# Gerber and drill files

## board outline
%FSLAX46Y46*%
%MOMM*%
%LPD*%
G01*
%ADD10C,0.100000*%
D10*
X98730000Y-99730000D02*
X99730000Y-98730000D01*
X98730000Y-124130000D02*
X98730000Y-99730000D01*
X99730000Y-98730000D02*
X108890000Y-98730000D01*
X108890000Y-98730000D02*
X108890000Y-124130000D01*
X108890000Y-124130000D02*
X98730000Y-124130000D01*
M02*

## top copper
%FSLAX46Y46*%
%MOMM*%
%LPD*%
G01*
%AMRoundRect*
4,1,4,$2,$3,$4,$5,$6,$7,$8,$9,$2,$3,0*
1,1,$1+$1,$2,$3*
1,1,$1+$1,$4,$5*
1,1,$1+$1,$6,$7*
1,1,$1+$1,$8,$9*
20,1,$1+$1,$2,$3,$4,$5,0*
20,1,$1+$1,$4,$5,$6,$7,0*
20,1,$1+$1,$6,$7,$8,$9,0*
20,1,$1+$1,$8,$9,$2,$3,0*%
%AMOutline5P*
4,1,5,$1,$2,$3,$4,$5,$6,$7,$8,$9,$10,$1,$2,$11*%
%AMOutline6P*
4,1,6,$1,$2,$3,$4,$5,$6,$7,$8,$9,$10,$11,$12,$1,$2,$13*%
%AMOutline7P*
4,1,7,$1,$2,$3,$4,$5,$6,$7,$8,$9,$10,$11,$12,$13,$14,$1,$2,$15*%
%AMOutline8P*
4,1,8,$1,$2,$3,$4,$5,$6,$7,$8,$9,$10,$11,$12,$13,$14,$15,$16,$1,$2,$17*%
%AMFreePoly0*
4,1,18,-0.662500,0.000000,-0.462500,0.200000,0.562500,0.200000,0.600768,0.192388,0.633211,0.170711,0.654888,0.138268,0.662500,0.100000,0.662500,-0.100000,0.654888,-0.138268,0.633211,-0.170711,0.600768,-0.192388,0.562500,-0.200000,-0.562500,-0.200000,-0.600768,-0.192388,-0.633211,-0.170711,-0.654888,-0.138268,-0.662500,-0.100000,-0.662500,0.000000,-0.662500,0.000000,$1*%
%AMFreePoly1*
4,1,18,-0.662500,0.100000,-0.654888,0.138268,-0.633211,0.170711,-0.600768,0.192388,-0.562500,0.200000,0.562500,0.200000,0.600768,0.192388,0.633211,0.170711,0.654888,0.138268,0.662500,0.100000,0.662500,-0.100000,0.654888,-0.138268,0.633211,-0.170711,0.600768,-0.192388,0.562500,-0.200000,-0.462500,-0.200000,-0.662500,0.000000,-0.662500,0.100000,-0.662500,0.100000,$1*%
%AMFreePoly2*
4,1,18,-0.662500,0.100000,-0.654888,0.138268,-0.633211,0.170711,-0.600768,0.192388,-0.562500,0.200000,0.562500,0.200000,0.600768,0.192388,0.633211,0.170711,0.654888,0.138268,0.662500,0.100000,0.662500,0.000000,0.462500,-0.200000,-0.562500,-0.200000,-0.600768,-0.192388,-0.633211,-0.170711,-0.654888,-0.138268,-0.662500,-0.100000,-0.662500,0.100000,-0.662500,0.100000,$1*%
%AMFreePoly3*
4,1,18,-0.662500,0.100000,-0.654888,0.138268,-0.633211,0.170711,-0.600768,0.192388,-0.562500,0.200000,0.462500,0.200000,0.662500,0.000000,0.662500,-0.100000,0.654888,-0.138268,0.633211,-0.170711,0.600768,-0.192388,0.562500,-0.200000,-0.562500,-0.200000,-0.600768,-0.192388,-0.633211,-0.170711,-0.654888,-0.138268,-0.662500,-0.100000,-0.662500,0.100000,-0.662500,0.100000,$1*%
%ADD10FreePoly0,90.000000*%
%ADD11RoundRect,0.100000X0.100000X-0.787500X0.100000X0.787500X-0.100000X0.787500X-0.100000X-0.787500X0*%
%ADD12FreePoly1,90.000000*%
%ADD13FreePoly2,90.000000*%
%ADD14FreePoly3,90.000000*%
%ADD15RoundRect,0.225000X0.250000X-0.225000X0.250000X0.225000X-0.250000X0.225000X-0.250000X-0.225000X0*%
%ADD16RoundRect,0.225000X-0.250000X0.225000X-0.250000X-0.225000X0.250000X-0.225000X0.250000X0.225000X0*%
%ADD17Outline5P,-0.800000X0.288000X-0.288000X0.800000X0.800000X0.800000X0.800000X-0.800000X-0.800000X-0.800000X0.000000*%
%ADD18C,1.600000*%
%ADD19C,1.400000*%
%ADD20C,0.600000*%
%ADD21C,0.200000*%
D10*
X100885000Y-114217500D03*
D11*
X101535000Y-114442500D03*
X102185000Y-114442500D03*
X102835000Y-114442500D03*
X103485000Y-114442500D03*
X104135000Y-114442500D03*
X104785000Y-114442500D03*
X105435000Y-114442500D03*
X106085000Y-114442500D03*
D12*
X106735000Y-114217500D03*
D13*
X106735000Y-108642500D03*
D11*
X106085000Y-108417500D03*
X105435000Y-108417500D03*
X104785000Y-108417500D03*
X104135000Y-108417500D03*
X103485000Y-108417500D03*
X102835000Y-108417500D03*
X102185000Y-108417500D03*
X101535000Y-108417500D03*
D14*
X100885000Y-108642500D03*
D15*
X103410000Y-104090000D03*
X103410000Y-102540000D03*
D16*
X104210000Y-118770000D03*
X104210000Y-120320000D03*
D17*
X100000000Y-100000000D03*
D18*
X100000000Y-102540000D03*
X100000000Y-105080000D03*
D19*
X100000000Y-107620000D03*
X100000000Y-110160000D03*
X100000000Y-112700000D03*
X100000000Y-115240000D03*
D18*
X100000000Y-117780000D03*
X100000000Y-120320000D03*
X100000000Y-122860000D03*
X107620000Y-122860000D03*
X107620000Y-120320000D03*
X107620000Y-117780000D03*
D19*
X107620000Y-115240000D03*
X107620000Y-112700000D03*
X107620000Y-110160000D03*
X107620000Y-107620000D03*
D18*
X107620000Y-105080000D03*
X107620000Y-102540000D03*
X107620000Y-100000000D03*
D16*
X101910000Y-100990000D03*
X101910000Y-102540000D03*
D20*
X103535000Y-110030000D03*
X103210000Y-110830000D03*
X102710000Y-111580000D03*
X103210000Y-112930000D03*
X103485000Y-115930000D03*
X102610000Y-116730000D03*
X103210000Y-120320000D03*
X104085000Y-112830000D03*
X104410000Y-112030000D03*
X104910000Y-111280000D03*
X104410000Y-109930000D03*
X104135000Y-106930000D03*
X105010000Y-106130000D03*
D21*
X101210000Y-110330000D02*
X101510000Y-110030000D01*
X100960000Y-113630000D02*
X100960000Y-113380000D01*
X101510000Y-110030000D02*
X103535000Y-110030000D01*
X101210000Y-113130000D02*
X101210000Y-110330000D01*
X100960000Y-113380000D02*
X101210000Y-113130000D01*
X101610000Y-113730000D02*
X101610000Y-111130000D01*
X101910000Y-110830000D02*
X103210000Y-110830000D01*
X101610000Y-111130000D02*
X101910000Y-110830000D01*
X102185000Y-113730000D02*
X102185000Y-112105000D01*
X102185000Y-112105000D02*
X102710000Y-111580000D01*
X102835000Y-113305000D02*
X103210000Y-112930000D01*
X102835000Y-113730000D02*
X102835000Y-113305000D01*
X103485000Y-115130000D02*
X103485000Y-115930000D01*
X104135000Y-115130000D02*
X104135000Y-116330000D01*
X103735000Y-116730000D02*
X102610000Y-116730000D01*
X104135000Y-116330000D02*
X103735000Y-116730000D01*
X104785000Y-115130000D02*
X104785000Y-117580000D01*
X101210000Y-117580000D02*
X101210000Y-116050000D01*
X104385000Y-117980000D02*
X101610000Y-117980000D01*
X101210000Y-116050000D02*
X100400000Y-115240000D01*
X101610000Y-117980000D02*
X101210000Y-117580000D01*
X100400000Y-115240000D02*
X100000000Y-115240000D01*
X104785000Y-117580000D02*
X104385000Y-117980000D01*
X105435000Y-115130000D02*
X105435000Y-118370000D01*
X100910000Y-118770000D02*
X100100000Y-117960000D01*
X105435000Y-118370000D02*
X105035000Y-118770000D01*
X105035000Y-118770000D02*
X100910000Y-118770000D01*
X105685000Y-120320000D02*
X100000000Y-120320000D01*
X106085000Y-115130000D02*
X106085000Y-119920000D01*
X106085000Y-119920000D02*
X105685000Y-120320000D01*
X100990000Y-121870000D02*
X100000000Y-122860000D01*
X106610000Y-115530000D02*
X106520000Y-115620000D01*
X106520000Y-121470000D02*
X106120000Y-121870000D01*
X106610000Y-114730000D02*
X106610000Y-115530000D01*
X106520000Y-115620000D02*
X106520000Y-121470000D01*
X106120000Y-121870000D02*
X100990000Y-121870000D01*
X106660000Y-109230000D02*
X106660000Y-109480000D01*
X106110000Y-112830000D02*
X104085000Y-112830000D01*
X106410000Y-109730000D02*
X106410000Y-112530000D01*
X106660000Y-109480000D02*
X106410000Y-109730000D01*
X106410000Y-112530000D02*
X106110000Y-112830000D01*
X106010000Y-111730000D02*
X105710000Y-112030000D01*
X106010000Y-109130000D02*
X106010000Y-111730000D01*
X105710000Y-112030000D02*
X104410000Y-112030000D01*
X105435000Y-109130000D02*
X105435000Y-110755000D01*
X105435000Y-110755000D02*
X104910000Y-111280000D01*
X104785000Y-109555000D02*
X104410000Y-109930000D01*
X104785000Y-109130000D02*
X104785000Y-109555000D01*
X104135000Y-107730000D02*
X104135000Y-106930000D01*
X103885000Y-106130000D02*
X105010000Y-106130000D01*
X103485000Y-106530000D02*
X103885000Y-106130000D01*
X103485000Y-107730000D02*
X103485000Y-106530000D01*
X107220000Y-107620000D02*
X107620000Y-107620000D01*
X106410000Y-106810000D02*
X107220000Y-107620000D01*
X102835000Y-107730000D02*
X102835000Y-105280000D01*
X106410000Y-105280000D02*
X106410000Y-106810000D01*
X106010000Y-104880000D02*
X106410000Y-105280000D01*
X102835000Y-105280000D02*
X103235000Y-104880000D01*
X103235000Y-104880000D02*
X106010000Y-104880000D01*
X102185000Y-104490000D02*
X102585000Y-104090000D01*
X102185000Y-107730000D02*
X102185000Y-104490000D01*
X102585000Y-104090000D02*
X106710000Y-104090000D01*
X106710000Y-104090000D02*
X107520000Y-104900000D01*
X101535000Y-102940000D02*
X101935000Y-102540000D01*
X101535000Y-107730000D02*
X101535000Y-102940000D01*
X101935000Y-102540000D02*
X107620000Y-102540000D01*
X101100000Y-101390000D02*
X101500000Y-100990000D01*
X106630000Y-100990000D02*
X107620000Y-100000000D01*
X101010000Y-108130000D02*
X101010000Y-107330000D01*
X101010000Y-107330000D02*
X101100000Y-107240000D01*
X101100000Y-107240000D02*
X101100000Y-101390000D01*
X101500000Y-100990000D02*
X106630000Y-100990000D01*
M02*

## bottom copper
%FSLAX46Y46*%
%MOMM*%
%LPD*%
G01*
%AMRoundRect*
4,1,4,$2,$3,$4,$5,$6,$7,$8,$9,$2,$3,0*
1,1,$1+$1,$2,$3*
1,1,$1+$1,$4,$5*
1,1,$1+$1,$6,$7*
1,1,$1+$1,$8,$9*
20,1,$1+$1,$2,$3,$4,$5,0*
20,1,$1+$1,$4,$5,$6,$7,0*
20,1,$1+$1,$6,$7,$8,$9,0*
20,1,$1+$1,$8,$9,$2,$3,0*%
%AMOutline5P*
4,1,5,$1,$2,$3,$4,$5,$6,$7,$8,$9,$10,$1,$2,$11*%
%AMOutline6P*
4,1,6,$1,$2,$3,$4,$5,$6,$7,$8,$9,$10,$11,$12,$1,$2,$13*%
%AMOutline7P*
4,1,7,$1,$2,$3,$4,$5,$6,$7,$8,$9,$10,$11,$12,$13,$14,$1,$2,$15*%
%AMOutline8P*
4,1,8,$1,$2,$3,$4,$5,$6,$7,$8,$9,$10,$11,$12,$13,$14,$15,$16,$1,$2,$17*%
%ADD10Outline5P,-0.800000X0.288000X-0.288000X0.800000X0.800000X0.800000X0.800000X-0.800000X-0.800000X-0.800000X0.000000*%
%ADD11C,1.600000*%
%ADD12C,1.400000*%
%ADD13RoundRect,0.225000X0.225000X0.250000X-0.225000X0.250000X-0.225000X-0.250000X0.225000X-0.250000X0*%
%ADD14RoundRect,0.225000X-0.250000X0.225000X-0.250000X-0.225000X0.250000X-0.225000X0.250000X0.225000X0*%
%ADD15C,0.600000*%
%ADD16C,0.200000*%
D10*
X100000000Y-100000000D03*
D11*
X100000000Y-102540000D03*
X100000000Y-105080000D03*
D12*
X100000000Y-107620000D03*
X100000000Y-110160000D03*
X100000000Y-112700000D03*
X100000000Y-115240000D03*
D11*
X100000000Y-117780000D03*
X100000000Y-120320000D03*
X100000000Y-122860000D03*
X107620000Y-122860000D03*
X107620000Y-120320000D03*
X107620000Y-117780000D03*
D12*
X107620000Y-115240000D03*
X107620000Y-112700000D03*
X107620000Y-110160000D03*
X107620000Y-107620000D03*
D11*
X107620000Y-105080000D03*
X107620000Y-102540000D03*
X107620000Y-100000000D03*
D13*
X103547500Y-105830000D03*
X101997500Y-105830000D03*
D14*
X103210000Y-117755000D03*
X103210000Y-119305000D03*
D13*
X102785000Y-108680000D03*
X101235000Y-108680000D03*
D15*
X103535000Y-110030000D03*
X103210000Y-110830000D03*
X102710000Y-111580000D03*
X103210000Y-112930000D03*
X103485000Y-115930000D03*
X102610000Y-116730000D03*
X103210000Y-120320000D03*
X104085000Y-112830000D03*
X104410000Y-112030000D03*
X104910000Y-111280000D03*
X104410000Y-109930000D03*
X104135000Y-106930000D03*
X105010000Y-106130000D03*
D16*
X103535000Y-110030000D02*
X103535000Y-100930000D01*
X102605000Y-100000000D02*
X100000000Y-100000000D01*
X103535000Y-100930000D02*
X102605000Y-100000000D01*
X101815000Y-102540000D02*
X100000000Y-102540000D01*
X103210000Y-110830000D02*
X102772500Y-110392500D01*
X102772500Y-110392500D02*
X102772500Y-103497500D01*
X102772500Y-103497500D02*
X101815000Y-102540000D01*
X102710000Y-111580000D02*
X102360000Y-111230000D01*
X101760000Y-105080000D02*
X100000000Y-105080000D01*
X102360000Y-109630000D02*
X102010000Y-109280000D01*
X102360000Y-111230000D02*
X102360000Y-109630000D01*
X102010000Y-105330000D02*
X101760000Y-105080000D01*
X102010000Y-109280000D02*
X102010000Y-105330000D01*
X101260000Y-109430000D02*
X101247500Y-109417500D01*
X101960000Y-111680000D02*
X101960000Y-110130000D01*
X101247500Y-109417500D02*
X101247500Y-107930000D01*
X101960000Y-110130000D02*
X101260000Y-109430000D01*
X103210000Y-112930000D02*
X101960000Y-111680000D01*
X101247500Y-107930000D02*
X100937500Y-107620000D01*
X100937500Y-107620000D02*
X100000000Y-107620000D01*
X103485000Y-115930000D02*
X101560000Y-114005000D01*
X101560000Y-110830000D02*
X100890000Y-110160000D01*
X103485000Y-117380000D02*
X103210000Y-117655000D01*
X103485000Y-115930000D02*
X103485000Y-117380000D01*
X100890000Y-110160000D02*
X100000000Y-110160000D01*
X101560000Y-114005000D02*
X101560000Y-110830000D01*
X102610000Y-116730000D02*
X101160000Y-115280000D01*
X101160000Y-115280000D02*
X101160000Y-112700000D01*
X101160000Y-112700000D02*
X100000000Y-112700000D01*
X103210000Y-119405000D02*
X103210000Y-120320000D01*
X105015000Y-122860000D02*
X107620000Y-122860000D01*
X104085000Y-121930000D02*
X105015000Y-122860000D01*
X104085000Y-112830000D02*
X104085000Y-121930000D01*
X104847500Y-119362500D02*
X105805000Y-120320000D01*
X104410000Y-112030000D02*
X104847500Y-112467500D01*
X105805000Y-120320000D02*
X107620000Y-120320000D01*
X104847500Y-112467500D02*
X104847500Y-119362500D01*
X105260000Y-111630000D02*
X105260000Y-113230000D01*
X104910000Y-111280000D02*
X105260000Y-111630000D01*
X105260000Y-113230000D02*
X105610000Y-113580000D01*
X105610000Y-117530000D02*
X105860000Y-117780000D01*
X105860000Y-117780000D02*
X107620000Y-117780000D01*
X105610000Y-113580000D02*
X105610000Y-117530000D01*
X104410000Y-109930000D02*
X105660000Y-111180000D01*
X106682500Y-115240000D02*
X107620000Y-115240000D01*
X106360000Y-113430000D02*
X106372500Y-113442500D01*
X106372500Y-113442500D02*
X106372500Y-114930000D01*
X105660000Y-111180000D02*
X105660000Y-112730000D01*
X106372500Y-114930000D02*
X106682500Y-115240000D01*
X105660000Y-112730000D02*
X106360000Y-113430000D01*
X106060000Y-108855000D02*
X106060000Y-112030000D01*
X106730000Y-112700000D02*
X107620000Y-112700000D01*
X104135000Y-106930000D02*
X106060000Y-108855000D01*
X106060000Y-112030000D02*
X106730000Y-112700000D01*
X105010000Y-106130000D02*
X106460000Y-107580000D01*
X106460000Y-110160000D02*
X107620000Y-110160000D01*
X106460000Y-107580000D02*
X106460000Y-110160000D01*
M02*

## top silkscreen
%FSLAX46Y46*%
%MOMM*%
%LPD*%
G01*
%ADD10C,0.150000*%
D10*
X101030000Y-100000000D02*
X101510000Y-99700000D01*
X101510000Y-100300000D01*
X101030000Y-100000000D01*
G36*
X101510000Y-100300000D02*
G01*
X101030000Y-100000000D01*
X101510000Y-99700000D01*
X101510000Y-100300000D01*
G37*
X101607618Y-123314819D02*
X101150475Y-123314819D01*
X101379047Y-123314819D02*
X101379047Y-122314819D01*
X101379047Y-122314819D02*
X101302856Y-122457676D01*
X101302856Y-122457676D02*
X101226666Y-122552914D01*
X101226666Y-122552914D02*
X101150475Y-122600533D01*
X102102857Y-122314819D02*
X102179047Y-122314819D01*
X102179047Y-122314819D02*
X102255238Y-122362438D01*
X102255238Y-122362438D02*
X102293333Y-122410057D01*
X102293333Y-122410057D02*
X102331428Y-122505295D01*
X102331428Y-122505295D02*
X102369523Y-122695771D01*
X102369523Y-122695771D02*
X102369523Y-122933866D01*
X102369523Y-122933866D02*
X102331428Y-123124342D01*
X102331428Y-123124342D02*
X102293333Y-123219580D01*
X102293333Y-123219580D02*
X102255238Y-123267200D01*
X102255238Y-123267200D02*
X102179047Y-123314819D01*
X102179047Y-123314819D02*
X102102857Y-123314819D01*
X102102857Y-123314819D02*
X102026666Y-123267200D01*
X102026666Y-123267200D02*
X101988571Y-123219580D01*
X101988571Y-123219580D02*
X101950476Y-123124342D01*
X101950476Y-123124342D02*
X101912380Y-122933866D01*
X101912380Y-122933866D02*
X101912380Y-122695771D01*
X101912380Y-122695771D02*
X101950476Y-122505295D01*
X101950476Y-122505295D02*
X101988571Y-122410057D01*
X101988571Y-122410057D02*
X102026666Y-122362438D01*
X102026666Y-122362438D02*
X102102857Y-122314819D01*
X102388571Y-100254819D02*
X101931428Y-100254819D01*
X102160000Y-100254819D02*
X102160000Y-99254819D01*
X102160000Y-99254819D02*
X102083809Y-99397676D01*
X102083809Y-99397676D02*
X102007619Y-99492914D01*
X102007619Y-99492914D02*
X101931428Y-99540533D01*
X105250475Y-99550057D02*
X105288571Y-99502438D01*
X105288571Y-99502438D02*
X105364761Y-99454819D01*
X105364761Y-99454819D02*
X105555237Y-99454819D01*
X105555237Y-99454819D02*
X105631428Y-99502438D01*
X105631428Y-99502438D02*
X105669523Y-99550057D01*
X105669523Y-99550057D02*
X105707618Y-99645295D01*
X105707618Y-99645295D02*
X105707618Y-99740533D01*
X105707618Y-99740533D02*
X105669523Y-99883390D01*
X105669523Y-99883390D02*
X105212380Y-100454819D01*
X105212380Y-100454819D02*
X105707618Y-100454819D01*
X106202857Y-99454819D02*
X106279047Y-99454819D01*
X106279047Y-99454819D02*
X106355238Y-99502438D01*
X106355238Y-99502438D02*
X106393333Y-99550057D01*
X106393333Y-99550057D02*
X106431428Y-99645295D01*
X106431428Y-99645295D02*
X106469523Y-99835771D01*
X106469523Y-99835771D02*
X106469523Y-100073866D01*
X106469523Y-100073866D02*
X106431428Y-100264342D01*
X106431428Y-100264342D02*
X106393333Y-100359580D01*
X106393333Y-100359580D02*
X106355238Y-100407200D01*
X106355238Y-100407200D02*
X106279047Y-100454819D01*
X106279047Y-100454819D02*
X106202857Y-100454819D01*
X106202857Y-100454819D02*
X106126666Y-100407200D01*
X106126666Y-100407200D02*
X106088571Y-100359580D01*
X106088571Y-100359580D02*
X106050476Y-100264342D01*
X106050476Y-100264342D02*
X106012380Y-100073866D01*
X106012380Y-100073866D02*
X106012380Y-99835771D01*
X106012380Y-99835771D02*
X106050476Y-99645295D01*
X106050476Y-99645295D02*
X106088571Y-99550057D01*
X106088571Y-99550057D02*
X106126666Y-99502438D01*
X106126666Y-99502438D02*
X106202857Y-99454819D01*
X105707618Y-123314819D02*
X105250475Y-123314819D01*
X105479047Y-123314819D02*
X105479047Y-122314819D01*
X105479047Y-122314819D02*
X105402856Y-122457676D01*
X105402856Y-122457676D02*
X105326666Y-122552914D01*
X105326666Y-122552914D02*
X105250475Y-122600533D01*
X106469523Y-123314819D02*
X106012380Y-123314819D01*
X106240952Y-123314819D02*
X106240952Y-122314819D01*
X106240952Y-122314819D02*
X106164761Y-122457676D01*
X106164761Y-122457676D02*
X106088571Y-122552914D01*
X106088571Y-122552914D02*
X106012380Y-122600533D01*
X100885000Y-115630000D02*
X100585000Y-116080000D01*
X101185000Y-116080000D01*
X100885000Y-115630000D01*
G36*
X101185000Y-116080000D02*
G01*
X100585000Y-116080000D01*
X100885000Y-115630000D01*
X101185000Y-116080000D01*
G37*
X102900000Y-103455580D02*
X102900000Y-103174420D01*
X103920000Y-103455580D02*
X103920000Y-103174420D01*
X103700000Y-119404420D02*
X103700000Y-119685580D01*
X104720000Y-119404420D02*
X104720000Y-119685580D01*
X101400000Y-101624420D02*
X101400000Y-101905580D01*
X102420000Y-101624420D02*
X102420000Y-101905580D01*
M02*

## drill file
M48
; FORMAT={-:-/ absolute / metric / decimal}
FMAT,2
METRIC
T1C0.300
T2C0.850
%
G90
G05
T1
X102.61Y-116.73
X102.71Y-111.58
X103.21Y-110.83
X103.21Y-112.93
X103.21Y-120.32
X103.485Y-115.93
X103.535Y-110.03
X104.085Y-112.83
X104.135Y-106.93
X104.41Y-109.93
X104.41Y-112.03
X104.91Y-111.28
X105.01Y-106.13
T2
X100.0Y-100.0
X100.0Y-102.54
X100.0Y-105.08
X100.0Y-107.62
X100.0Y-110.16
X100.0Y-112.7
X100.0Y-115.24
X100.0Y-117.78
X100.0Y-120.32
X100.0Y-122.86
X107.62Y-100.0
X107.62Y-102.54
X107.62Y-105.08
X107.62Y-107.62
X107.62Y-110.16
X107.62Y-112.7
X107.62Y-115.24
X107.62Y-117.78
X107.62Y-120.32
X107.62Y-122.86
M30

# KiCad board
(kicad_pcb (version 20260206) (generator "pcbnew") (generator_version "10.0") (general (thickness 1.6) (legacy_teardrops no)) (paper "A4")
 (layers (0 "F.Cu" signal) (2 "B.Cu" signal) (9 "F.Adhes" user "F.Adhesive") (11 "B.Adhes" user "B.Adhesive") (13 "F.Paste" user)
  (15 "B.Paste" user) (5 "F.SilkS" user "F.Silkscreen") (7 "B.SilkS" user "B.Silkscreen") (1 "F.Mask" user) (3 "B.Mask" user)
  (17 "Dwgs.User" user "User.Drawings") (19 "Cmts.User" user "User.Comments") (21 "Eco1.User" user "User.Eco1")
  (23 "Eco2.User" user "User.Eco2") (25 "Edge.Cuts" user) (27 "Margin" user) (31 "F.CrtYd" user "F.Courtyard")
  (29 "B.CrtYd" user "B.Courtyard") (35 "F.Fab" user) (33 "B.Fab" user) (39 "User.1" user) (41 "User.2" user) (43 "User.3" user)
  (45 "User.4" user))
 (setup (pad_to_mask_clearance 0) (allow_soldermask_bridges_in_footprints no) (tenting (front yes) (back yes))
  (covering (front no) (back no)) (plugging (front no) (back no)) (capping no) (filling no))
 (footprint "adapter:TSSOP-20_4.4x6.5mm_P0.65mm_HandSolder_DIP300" (layer "F.Cu") (at 103.81 111.43 90)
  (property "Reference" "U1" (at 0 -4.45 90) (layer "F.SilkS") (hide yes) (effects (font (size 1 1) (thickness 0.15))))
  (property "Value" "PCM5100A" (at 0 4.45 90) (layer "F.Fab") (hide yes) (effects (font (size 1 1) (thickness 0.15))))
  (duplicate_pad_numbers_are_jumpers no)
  (fp_poly (pts (xy -4.2 -2.925) (xy -4.65 -3.225) (xy -4.65 -2.625)) (stroke (width 0.15) (type solid)) (fill yes) (layer "F.SilkS"))
  (pad "1" smd roundrect (at -2.7875 -2.925 90) (size 1.325 0.4) (layers "F.Cu" "F.Mask" "F.Paste") (roundrect_rratio 0.25)
   (chamfer_ratio 0.5) (chamfer top_left) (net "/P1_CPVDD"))
  (pad "2" smd roundrect (at -3.0125 -2.275 90) (size 1.775 0.4) (layers "F.Cu" "F.Mask" "F.Paste") (roundrect_rratio 0.25) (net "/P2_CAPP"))
  (pad "3" smd roundrect (at -3.0125 -1.625 90) (size 1.775 0.4) (layers "F.Cu" "F.Mask" "F.Paste") (roundrect_rratio 0.25)
   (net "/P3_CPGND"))
  (pad "4" smd roundrect (at -3.0125 -0.975 90) (size 1.775 0.4) (layers "F.Cu" "F.Mask" "F.Paste") (roundrect_rratio 0.25) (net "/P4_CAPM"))
  (pad "5" smd roundrect (at -3.0125 -0.325 90) (size 1.775 0.4) (layers "F.Cu" "F.Mask" "F.Paste") (roundrect_rratio 0.25) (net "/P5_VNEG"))
  (pad "6" smd roundrect (at -3.0125 0.325 90) (size 1.775 0.4) (layers "F.Cu" "F.Mask" "F.Paste") (roundrect_rratio 0.25) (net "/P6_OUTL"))
  (pad "7" smd roundrect (at -3.0125 0.975 90) (size 1.775 0.4) (layers "F.Cu" "F.Mask" "F.Paste") (roundrect_rratio 0.25) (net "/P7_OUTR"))
  (pad "8" smd roundrect (at -3.0125 1.625 90) (size 1.775 0.4) (layers "F.Cu" "F.Mask" "F.Paste") (roundrect_rratio 0.25) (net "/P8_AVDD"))
  (pad "9" smd roundrect (at -3.0125 2.275 90) (size 1.775 0.4) (layers "F.Cu" "F.Mask" "F.Paste") (roundrect_rratio 0.25) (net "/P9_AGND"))
  (pad "10" smd roundrect (at -2.7875 2.925 90) (size 1.325 0.4) (layers "F.Cu" "F.Mask" "F.Paste") (roundrect_rratio 0.25)
   (chamfer_ratio 0.5) (chamfer bottom_left) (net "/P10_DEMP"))
  (pad "11" smd roundrect (at 2.7875 2.925 90) (size 1.325 0.4) (layers "F.Cu" "F.Mask" "F.Paste") (roundrect_rratio 0.25)
   (chamfer_ratio 0.5) (chamfer bottom_right) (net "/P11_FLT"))
  (pad "12" smd roundrect (at 3.0125 2.275 90) (size 1.775 0.4) (layers "F.Cu" "F.Mask" "F.Paste") (roundrect_rratio 0.25) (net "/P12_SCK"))
  (pad "13" smd roundrect (at 3.0125 1.625 90) (size 1.775 0.4) (layers "F.Cu" "F.Mask" "F.Paste") (roundrect_rratio 0.25) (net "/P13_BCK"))
  (pad "14" smd roundrect (at 3.0125 0.975 90) (size 1.775 0.4) (layers "F.Cu" "F.Mask" "F.Paste") (roundrect_rratio 0.25) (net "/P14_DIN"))
  (pad "15" smd roundrect (at 3.0125 0.325 90) (size 1.775 0.4) (layers "F.Cu" "F.Mask" "F.Paste") (roundrect_rratio 0.25) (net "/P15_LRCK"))
  (pad "16" smd roundrect (at 3.0125 -0.325 90) (size 1.775 0.4) (layers "F.Cu" "F.Mask" "F.Paste") (roundrect_rratio 0.25) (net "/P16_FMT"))
  (pad "17" smd roundrect (at 3.0125 -0.975 90) (size 1.775 0.4) (layers "F.Cu" "F.Mask" "F.Paste") (roundrect_rratio 0.25)
   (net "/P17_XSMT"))
  (pad "18" smd roundrect (at 3.0125 -1.625 90) (size 1.775 0.4) (layers "F.Cu" "F.Mask" "F.Paste") (roundrect_rratio 0.25)
   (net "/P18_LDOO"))
  (pad "19" smd roundrect (at 3.0125 -2.275 90) (size 1.775 0.4) (layers "F.Cu" "F.Mask" "F.Paste") (roundrect_rratio 0.25)
   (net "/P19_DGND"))
  (pad "20" smd roundrect (at 2.7875 -2.925 90) (size 1.325 0.4) (layers "F.Cu" "F.Mask" "F.Paste") (roundrect_rratio 0.25)
   (chamfer_ratio 0.5) (chamfer top_right) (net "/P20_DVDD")))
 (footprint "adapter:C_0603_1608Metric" (layer "F.Cu") (at 103.41 103.315 90)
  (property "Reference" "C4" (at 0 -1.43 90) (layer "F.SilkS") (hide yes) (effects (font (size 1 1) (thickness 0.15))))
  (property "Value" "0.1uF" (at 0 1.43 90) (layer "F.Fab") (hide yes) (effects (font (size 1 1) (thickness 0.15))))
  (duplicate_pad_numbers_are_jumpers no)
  (fp_line (start -0.14058 -0.51) (end 0.14058 -0.51) (stroke (width 0.15) (type solid)) (layer "F.SilkS"))
  (fp_line (start -0.14058 0.51) (end 0.14058 0.51) (stroke (width 0.15) (type solid)) (layer "F.SilkS"))
  (pad "1" smd roundrect (at -0.775 0 90) (size 0.9 0.95) (layers "F.Cu" "F.Mask" "F.Paste") (roundrect_rratio 0.25) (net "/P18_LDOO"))
  (pad "2" smd roundrect (at 0.775 0 90) (size 0.9 0.95) (layers "F.Cu" "F.Mask" "F.Paste") (roundrect_rratio 0.25) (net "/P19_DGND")))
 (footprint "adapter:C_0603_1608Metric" (layer "F.Cu") (at 104.21 119.545 -90)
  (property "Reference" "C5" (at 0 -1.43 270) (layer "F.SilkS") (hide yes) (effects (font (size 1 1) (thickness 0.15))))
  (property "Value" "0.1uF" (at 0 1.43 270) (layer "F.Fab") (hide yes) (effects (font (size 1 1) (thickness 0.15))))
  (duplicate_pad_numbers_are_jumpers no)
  (fp_line (start -0.14058 0.51) (end 0.14058 0.51) (stroke (width 0.15) (type solid)) (layer "F.SilkS"))
  (fp_line (start -0.14058 -0.51) (end 0.14058 -0.51) (stroke (width 0.15) (type solid)) (layer "F.SilkS"))
  (pad "1" smd roundrect (at -0.775 0 270) (size 0.9 0.95) (layers "F.Cu" "F.Mask" "F.Paste") (roundrect_rratio 0.25) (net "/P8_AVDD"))
  (pad "2" smd roundrect (at 0.775 0 270) (size 0.9 0.95) (layers "F.Cu" "F.Mask" "F.Paste") (roundrect_rratio 0.25) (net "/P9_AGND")))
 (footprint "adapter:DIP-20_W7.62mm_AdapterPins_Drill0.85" (layer "F.Cu") (at 100 100)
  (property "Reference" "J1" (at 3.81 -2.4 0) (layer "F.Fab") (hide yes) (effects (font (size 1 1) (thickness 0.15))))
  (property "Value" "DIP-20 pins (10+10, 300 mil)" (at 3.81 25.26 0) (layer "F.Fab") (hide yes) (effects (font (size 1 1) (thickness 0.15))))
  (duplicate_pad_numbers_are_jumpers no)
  (pad "1" thru_hole roundrect (at 0 0) (size 1.6 1.6) (drill 0.85) (layers "*.Cu" "*.Mask") (remove_unused_layers no) (roundrect_rratio 0)
   (chamfer_ratio 0.32) (chamfer top_left) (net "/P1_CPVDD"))
  (pad "2" thru_hole circle (at 0 2.54) (size 1.6 1.6) (drill 0.85) (layers "*.Cu" "*.Mask") (remove_unused_layers no) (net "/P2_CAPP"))
  (pad "3" thru_hole circle (at 0 5.08) (size 1.6 1.6) (drill 0.85) (layers "*.Cu" "*.Mask") (remove_unused_layers no) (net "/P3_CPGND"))
  (pad "4" thru_hole circle (at 0 7.62) (size 1.4 1.4) (drill 0.85) (layers "*.Cu" "*.Mask") (remove_unused_layers no) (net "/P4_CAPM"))
  (pad "5" thru_hole circle (at 0 10.16) (size 1.4 1.4) (drill 0.85) (layers "*.Cu" "*.Mask") (remove_unused_layers no) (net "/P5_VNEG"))
  (pad "6" thru_hole circle (at 0 12.7) (size 1.4 1.4) (drill 0.85) (layers "*.Cu" "*.Mask") (remove_unused_layers no) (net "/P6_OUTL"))
  (pad "7" thru_hole circle (at 0 15.24) (size 1.4 1.4) (drill 0.85) (layers "*.Cu" "*.Mask") (remove_unused_layers no) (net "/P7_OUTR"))
  (pad "8" thru_hole circle (at 0 17.78) (size 1.6 1.6) (drill 0.85) (layers "*.Cu" "*.Mask") (remove_unused_layers no) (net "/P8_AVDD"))
  (pad "9" thru_hole circle (at 0 20.32) (size 1.6 1.6) (drill 0.85) (layers "*.Cu" "*.Mask") (remove_unused_layers no) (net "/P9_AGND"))
  (pad "10" thru_hole circle (at 0 22.86) (size 1.6 1.6) (drill 0.85) (layers "*.Cu" "*.Mask") (remove_unused_layers no) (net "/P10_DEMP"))
  (pad "11" thru_hole circle (at 7.62 22.86) (size 1.6 1.6) (drill 0.85) (layers "*.Cu" "*.Mask") (remove_unused_layers no) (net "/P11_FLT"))
  (pad "12" thru_hole circle (at 7.62 20.32) (size 1.6 1.6) (drill 0.85) (layers "*.Cu" "*.Mask") (remove_unused_layers no) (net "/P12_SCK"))
  (pad "13" thru_hole circle (at 7.62 17.78) (size 1.6 1.6) (drill 0.85) (layers "*.Cu" "*.Mask") (remove_unused_layers no) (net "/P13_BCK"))
  (pad "14" thru_hole circle (at 7.62 15.24) (size 1.4 1.4) (drill 0.85) (layers "*.Cu" "*.Mask") (remove_unused_layers no) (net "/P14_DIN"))
  (pad "15" thru_hole circle (at 7.62 12.7) (size 1.4 1.4) (drill 0.85) (layers "*.Cu" "*.Mask") (remove_unused_layers no) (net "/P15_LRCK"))
  (pad "16" thru_hole circle (at 7.62 10.16) (size 1.4 1.4) (drill 0.85) (layers "*.Cu" "*.Mask") (remove_unused_layers no) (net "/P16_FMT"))
  (pad "17" thru_hole circle (at 7.62 7.62) (size 1.4 1.4) (drill 0.85) (layers "*.Cu" "*.Mask") (remove_unused_layers no) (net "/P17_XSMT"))
  (pad "18" thru_hole circle (at 7.62 5.08) (size 1.6 1.6) (drill 0.85) (layers "*.Cu" "*.Mask") (remove_unused_layers no) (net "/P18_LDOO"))
  (pad "19" thru_hole circle (at 7.62 2.54) (size 1.6 1.6) (drill 0.85) (layers "*.Cu" "*.Mask") (remove_unused_layers no) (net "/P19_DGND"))
  (pad "20" thru_hole circle (at 7.62 0) (size 1.6 1.6) (drill 0.85) (layers "*.Cu" "*.Mask") (remove_unused_layers no) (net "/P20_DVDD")))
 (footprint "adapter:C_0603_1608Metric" (layer "F.Cu") (at 101.91 101.765 -90)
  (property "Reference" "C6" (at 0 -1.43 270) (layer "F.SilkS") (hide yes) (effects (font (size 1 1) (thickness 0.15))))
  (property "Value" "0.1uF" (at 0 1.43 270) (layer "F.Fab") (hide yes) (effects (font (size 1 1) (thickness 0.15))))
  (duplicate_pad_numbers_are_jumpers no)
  (fp_line (start -0.14058 0.51) (end 0.14058 0.51) (stroke (width 0.15) (type solid)) (layer "F.SilkS"))
  (fp_line (start -0.14058 -0.51) (end 0.14058 -0.51) (stroke (width 0.15) (type solid)) (layer "F.SilkS"))
  (pad "1" smd roundrect (at -0.775 0 270) (size 0.9 0.95) (layers "F.Cu" "F.Mask" "F.Paste") (roundrect_rratio 0.25) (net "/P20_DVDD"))
  (pad "2" smd roundrect (at 0.775 0 270) (size 0.9 0.95) (layers "F.Cu" "F.Mask" "F.Paste") (roundrect_rratio 0.25) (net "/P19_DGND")))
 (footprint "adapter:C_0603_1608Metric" (layer "B.Cu") (at 102.7725 105.83 180)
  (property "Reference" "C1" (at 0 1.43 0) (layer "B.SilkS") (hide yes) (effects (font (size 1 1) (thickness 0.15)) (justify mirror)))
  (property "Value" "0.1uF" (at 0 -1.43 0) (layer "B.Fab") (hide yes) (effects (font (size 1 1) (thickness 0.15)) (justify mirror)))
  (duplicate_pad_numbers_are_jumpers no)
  (pad "1" smd roundrect (at -0.775 0 180) (size 0.9 0.95) (layers "B.Cu" "B.Mask" "B.Paste") (roundrect_rratio 0.25) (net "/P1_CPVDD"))
  (pad "2" smd roundrect (at 0.775 0 180) (size 0.9 0.95) (layers "B.Cu" "B.Mask" "B.Paste") (roundrect_rratio 0.25) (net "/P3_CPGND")))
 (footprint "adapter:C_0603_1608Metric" (layer "B.Cu") (at 103.21 118.53 -90)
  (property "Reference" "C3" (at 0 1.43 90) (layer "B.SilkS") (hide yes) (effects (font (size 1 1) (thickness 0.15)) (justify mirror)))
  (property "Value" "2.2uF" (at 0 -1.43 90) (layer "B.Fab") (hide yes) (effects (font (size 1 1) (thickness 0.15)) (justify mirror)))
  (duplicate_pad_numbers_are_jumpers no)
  (pad "1" smd roundrect (at -0.775 0 270) (size 0.9 0.95) (layers "B.Cu" "B.Mask" "B.Paste") (roundrect_rratio 0.25) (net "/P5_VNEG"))
  (pad "2" smd roundrect (at 0.775 0 270) (size 0.9 0.95) (layers "B.Cu" "B.Mask" "B.Paste") (roundrect_rratio 0.25) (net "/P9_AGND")))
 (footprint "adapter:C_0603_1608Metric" (layer "B.Cu") (at 102.01 108.68 180)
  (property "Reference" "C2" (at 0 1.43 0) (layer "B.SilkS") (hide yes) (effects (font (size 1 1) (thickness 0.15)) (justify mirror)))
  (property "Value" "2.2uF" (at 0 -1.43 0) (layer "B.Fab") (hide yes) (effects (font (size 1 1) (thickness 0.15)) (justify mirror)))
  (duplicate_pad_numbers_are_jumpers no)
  (pad "1" smd roundrect (at -0.775 0 180) (size 0.9 0.95) (layers "B.Cu" "B.Mask" "B.Paste") (roundrect_rratio 0.25) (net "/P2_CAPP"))
  (pad "2" smd roundrect (at 0.775 0 180) (size 0.9 0.95) (layers "B.Cu" "B.Mask" "B.Paste") (roundrect_rratio 0.25) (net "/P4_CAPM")))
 (gr_poly (pts (xy 101.03 100) (xy 101.51 99.7) (xy 101.51 100.3)) (stroke (width 0.15) (type default)) (fill yes) (layer "F.SilkS"))
 (gr_line (start 98.73 99.73) (end 99.73 98.73) (stroke (width 0.1) (type default)) (layer "Edge.Cuts"))
 (gr_line (start 98.73 124.13) (end 98.73 99.73) (stroke (width 0.1) (type default)) (layer "Edge.Cuts"))
 (gr_line (start 99.73 98.73) (end 108.89 98.73) (stroke (width 0.1) (type default)) (layer "Edge.Cuts"))
 (gr_line (start 108.89 98.73) (end 108.89 124.13) (stroke (width 0.1) (type default)) (layer "Edge.Cuts"))
 (gr_line (start 108.89 124.13) (end 98.73 124.13) (stroke (width 0.1) (type default)) (layer "Edge.Cuts"))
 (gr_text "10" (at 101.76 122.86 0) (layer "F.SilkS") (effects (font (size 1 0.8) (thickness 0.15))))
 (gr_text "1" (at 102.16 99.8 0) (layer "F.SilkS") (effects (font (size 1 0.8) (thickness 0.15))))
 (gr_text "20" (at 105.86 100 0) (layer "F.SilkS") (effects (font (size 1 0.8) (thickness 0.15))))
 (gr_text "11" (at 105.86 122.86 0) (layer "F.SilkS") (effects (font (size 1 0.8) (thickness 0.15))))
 (segment (start 101.21 110.33) (end 101.51 110.03) (width 0.2) (layer "F.Cu") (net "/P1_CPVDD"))
 (segment (start 100.96 113.63) (end 100.96 113.38) (width 0.2) (layer "F.Cu") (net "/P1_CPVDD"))
 (segment (start 101.51 110.03) (end 103.535 110.03) (width 0.2) (layer "F.Cu") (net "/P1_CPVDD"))
 (segment (start 101.21 113.13) (end 101.21 110.33) (width 0.2) (layer "F.Cu") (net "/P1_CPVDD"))
 (segment (start 100.96 113.38) (end 101.21 113.13) (width 0.2) (layer "F.Cu") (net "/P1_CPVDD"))
 (via (at 103.535 110.03) (size 0.6) (drill 0.3) (layers "F.Cu" "B.Cu") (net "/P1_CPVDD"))
 (segment (start 103.535 110.03) (end 103.535 100.93) (width 0.2) (layer "B.Cu") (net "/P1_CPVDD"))
 (segment (start 102.605 100) (end 100 100) (width 0.2) (layer "B.Cu") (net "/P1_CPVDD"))
 (segment (start 103.535 100.93) (end 102.605 100) (width 0.2) (layer "B.Cu") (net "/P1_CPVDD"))
 (segment (start 101.61 113.73) (end 101.61 111.13) (width 0.2) (layer "F.Cu") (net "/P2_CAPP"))
 (segment (start 101.91 110.83) (end 103.21 110.83) (width 0.2) (layer "F.Cu") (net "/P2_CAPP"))
 (segment (start 101.61 111.13) (end 101.91 110.83) (width 0.2) (layer "F.Cu") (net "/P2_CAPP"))
 (via (at 103.21 110.83) (size 0.6) (drill 0.3) (layers "F.Cu" "B.Cu") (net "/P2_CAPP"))
 (segment (start 101.815 102.54) (end 100 102.54) (width 0.2) (layer "B.Cu") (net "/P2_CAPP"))
 (segment (start 103.21 110.83) (end 102.7725 110.3925) (width 0.2) (layer "B.Cu") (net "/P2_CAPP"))
 (segment (start 102.7725 110.3925) (end 102.7725 103.4975) (width 0.2) (layer "B.Cu") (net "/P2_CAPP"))
 (segment (start 102.7725 103.4975) (end 101.815 102.54) (width 0.2) (layer "B.Cu") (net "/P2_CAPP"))
 (segment (start 102.185 113.73) (end 102.185 112.105) (width 0.2) (layer "F.Cu") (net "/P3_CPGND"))
 (segment (start 102.185 112.105) (end 102.71 111.58) (width 0.2) (layer "F.Cu") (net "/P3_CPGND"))
 (via (at 102.71 111.58) (size 0.6) (drill 0.3) (layers "F.Cu" "B.Cu") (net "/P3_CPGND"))
 (segment (start 102.71 111.58) (end 102.36 111.23) (width 0.2) (layer "B.Cu") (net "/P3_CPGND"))
 (segment (start 101.76 105.08) (end 100 105.08) (width 0.2) (layer "B.Cu") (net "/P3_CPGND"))
 (segment (start 102.36 109.63) (end 102.01 109.28) (width 0.2) (layer "B.Cu") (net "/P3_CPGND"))
 (segment (start 102.36 111.23) (end 102.36 109.63) (width 0.2) (layer "B.Cu") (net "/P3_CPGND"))
 (segment (start 102.01 105.33) (end 101.76 105.08) (width 0.2) (layer "B.Cu") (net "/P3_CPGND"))
 (segment (start 102.01 109.28) (end 102.01 105.33) (width 0.2) (layer "B.Cu") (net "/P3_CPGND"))
 (segment (start 102.835 113.305) (end 103.21 112.93) (width 0.2) (layer "F.Cu") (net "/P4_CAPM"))
 (segment (start 102.835 113.73) (end 102.835 113.305) (width 0.2) (layer "F.Cu") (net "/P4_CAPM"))
 (via (at 103.21 112.93) (size 0.6) (drill 0.3) (layers "F.Cu" "B.Cu") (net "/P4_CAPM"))
 (segment (start 101.26 109.43) (end 101.2475 109.4175) (width 0.2) (layer "B.Cu") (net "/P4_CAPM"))
 (segment (start 101.96 111.68) (end 101.96 110.13) (width 0.2) (layer "B.Cu") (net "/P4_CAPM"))
 (segment (start 101.2475 109.4175) (end 101.2475 107.93) (width 0.2) (layer "B.Cu") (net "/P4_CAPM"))
 (segment (start 101.96 110.13) (end 101.26 109.43) (width 0.2) (layer "B.Cu") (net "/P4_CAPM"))
 (segment (start 103.21 112.93) (end 101.96 111.68) (width 0.2) (layer "B.Cu") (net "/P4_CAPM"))
 (segment (start 101.2475 107.93) (end 100.9375 107.62) (width 0.2) (layer "B.Cu") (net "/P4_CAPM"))
 (segment (start 100.9375 107.62) (end 100 107.62) (width 0.2) (layer "B.Cu") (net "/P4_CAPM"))
 (segment (start 103.485 115.13) (end 103.485 115.93) (width 0.2) (layer "F.Cu") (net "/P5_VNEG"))
 (via (at 103.485 115.93) (size 0.6) (drill 0.3) (layers "F.Cu" "B.Cu") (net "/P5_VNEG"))
 (segment (start 103.485 115.93) (end 101.56 114.005) (width 0.2) (layer "B.Cu") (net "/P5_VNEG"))
 (segment (start 101.56 110.83) (end 100.89 110.16) (width 0.2) (layer "B.Cu") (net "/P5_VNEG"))
 (segment (start 103.485 117.38) (end 103.21 117.655) (width 0.2) (layer "B.Cu") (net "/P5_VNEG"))
 (segment (start 103.485 115.93) (end 103.485 117.38) (width 0.2) (layer "B.Cu") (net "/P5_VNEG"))
 (segment (start 100.89 110.16) (end 100 110.16) (width 0.2) (layer "B.Cu") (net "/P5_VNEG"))
 (segment (start 101.56 114.005) (end 101.56 110.83) (width 0.2) (layer "B.Cu") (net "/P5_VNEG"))
 (segment (start 104.135 115.13) (end 104.135 116.33) (width 0.2) (layer "F.Cu") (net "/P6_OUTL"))
 (segment (start 103.735 116.73) (end 102.61 116.73) (width 0.2) (layer "F.Cu") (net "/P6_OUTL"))
 (segment (start 104.135 116.33) (end 103.735 116.73) (width 0.2) (layer "F.Cu") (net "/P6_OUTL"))
 (via (at 102.61 116.73) (size 0.6) (drill 0.3) (layers "F.Cu" "B.Cu") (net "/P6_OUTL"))
 (segment (start 102.61 116.73) (end 101.16 115.28) (width 0.2) (layer "B.Cu") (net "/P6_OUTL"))
 (segment (start 101.16 115.28) (end 101.16 112.7) (width 0.2) (layer "B.Cu") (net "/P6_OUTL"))
 (segment (start 101.16 112.7) (end 100 112.7) (width 0.2) (layer "B.Cu") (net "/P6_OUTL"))
 (segment (start 104.785 115.13) (end 104.785 117.58) (width 0.2) (layer "F.Cu") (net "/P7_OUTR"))
 (segment (start 101.21 117.58) (end 101.21 116.05) (width 0.2) (layer "F.Cu") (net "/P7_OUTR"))
 (segment (start 104.385 117.98) (end 101.61 117.98) (width 0.2) (layer "F.Cu") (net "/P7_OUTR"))
 (segment (start 101.21 116.05) (end 100.4 115.24) (width 0.2) (layer "F.Cu") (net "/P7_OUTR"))
 (segment (start 101.61 117.98) (end 101.21 117.58) (width 0.2) (layer "F.Cu") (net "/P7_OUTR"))
 (segment (start 100.4 115.24) (end 100 115.24) (width 0.2) (layer "F.Cu") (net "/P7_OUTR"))
 (segment (start 104.785 117.58) (end 104.385 117.98) (width 0.2) (layer "F.Cu") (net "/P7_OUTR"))
 (segment (start 105.435 115.13) (end 105.435 118.37) (width 0.2) (layer "F.Cu") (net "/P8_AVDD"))
 (segment (start 100.91 118.77) (end 100.1 117.96) (width 0.2) (layer "F.Cu") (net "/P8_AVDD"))
 (segment (start 105.435 118.37) (end 105.035 118.77) (width 0.2) (layer "F.Cu") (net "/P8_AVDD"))
 (segment (start 105.035 118.77) (end 100.91 118.77) (width 0.2) (layer "F.Cu") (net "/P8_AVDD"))
 (segment (start 105.685 120.32) (end 100 120.32) (width 0.2) (layer "F.Cu") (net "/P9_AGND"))
 (segment (start 106.085 115.13) (end 106.085 119.92) (width 0.2) (layer "F.Cu") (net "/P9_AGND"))
 (segment (start 106.085 119.92) (end 105.685 120.32) (width 0.2) (layer "F.Cu") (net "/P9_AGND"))
 (via (at 103.21 120.32) (size 0.6) (drill 0.3) (layers "F.Cu" "B.Cu") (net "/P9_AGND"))
 (segment (start 103.21 119.405) (end 103.21 120.32) (width 0.2) (layer "B.Cu") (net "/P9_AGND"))
 (segment (start 100.99 121.87) (end 100 122.86) (width 0.2) (layer "F.Cu") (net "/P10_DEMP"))
 (segment (start 106.61 115.53) (end 106.52 115.62) (width 0.2) (layer "F.Cu") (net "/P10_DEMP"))
 (segment (start 106.52 121.47) (end 106.12 121.87) (width 0.2) (layer "F.Cu") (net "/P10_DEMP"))
 (segment (start 106.61 114.73) (end 106.61 115.53) (width 0.2) (layer "F.Cu") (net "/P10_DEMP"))
 (segment (start 106.52 115.62) (end 106.52 121.47) (width 0.2) (layer "F.Cu") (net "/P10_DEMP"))
 (segment (start 106.12 121.87) (end 100.99 121.87) (width 0.2) (layer "F.Cu") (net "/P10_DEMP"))
 (segment (start 106.66 109.23) (end 106.66 109.48) (width 0.2) (layer "F.Cu") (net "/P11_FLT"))
 (segment (start 106.11 112.83) (end 104.085 112.83) (width 0.2) (layer "F.Cu") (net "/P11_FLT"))
 (segment (start 106.41 109.73) (end 106.41 112.53) (width 0.2) (layer "F.Cu") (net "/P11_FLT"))
 (segment (start 106.66 109.48) (end 106.41 109.73) (width 0.2) (layer "F.Cu") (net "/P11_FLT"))
 (segment (start 106.41 112.53) (end 106.11 112.83) (width 0.2) (layer "F.Cu") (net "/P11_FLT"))
 (via (at 104.085 112.83) (size 0.6) (drill 0.3) (layers "F.Cu" "B.Cu") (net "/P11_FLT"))
 (segment (start 105.015 122.86) (end 107.62 122.86) (width 0.2) (layer "B.Cu") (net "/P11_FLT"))
 (segment (start 104.085 121.93) (end 105.015 122.86) (width 0.2) (layer "B.Cu") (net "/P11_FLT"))
 (segment (start 104.085 112.83) (end 104.085 121.93) (width 0.2) (layer "B.Cu") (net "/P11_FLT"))
 (segment (start 106.01 111.73) (end 105.71 112.03) (width 0.2) (layer "F.Cu") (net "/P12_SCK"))
 (segment (start 106.01 109.13) (end 106.01 111.73) (width 0.2) (layer "F.Cu") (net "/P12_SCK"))
 (segment (start 105.71 112.03) (end 104.41 112.03) (width 0.2) (layer "F.Cu") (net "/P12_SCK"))
 (via (at 104.41 112.03) (size 0.6) (drill 0.3) (layers "F.Cu" "B.Cu") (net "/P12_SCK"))
 (segment (start 104.8475 119.3625) (end 105.805 120.32) (width 0.2) (layer "B.Cu") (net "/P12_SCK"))
 (segment (start 104.41 112.03) (end 104.8475 112.4675) (width 0.2) (layer "B.Cu") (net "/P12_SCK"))
 (segment (start 105.805 120.32) (end 107.62 120.32) (width 0.2) (layer "B.Cu") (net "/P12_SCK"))
 (segment (start 104.8475 112.4675) (end 104.8475 119.3625) (width 0.2) (layer "B.Cu") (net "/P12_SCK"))
 (segment (start 105.435 109.13) (end 105.435 110.755) (width 0.2) (layer "F.Cu") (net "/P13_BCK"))
 (segment (start 105.435 110.755) (end 104.91 111.28) (width 0.2) (layer "F.Cu") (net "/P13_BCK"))
 (via (at 104.91 111.28) (size 0.6) (drill 0.3) (layers "F.Cu" "B.Cu") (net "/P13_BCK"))
 (segment (start 105.26 111.63) (end 105.26 113.23) (width 0.2) (layer "B.Cu") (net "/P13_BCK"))
 (segment (start 104.91 111.28) (end 105.26 111.63) (width 0.2) (layer "B.Cu") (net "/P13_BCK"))
 (segment (start 105.26 113.23) (end 105.61 113.58) (width 0.2) (layer "B.Cu") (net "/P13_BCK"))
 (segment (start 105.61 117.53) (end 105.86 117.78) (width 0.2) (layer "B.Cu") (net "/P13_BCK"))
 (segment (start 105.86 117.78) (end 107.62 117.78) (width 0.2) (layer "B.Cu") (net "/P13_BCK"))
 (segment (start 105.61 113.58) (end 105.61 117.53) (width 0.2) (layer "B.Cu") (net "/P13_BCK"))
 (segment (start 104.785 109.555) (end 104.41 109.93) (width 0.2) (layer "F.Cu") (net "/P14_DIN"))
 (segment (start 104.785 109.13) (end 104.785 109.555) (width 0.2) (layer "F.Cu") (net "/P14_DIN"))
 (via (at 104.41 109.93) (size 0.6) (drill 0.3) (layers "F.Cu" "B.Cu") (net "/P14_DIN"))
 (segment (start 104.41 109.93) (end 105.66 111.18) (width 0.2) (layer "B.Cu") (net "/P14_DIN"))
 (segment (start 106.6825 115.24) (end 107.62 115.24) (width 0.2) (layer "B.Cu") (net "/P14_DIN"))
 (segment (start 106.36 113.43) (end 106.3725 113.4425) (width 0.2) (layer "B.Cu") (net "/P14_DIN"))
 (segment (start 106.3725 113.4425) (end 106.3725 114.93) (width 0.2) (layer "B.Cu") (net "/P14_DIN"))
 (segment (start 105.66 111.18) (end 105.66 112.73) (width 0.2) (layer "B.Cu") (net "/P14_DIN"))
 (segment (start 106.3725 114.93) (end 106.6825 115.24) (width 0.2) (layer "B.Cu") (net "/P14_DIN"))
 (segment (start 105.66 112.73) (end 106.36 113.43) (width 0.2) (layer "B.Cu") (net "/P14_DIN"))
 (segment (start 104.135 107.73) (end 104.135 106.93) (width 0.2) (layer "F.Cu") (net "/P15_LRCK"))
 (via (at 104.135 106.93) (size 0.6) (drill 0.3) (layers "F.Cu" "B.Cu") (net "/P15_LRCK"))
 (segment (start 106.06 108.855) (end 106.06 112.03) (width 0.2) (layer "B.Cu") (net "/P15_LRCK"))
 (segment (start 106.73 112.7) (end 107.62 112.7) (width 0.2) (layer "B.Cu") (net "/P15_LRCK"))
 (segment (start 104.135 106.93) (end 106.06 108.855) (width 0.2) (layer "B.Cu") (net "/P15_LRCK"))
 (segment (start 106.06 112.03) (end 106.73 112.7) (width 0.2) (layer "B.Cu") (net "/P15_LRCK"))
 (segment (start 103.885 106.13) (end 105.01 106.13) (width 0.2) (layer "F.Cu") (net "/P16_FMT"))
 (segment (start 103.485 106.53) (end 103.885 106.13) (width 0.2) (layer "F.Cu") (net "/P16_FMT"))
 (segment (start 103.485 107.73) (end 103.485 106.53) (width 0.2) (layer "F.Cu") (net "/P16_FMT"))
 (via (at 105.01 106.13) (size 0.6) (drill 0.3) (layers "F.Cu" "B.Cu") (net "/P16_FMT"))
 (segment (start 105.01 106.13) (end 106.46 107.58) (width 0.2) (layer "B.Cu") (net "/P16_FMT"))
 (segment (start 106.46 110.16) (end 107.62 110.16) (width 0.2) (layer "B.Cu") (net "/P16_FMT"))
 (segment (start 106.46 107.58) (end 106.46 110.16) (width 0.2) (layer "B.Cu") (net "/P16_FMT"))
 (segment (start 107.22 107.62) (end 107.62 107.62) (width 0.2) (layer "F.Cu") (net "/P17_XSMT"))
 (segment (start 106.41 106.81) (end 107.22 107.62) (width 0.2) (layer "F.Cu") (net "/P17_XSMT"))
 (segment (start 102.835 107.73) (end 102.835 105.28) (width 0.2) (layer "F.Cu") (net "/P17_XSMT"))
 (segment (start 106.41 105.28) (end 106.41 106.81) (width 0.2) (layer "F.Cu") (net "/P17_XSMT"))
 (segment (start 106.01 104.88) (end 106.41 105.28) (width 0.2) (layer "F.Cu") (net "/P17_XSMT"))
 (segment (start 102.835 105.28) (end 103.235 104.88) (width 0.2) (layer "F.Cu") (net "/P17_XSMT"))
 (segment (start 103.235 104.88) (end 106.01 104.88) (width 0.2) (layer "F.Cu") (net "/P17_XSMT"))
 (segment (start 102.185 104.49) (end 102.585 104.09) (width 0.2) (layer "F.Cu") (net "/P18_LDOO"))
 (segment (start 102.185 107.73) (end 102.185 104.49) (width 0.2) (layer "F.Cu") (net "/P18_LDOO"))
 (segment (start 102.585 104.09) (end 106.71 104.09) (width 0.2) (layer "F.Cu") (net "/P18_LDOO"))
 (segment (start 106.71 104.09) (end 107.52 104.9) (width 0.2) (layer "F.Cu") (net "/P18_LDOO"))
 (segment (start 101.535 102.94) (end 101.935 102.54) (width 0.2) (layer "F.Cu") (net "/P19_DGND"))
 (segment (start 101.535 107.73) (end 101.535 102.94) (width 0.2) (layer "F.Cu") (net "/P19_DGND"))
 (segment (start 101.935 102.54) (end 107.62 102.54) (width 0.2) (layer "F.Cu") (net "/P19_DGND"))
 (segment (start 101.1 101.39) (end 101.5 100.99) (width 0.2) (layer "F.Cu") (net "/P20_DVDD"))
 (segment (start 106.63 100.99) (end 107.62 100) (width 0.2) (layer "F.Cu") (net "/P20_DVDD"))
 (segment (start 101.01 108.13) (end 101.01 107.33) (width 0.2) (layer "F.Cu") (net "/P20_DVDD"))
 (segment (start 101.01 107.33) (end 101.1 107.24) (width 0.2) (layer "F.Cu") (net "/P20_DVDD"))
 (segment (start 101.1 107.24) (end 101.1 101.39) (width 0.2) (layer "F.Cu") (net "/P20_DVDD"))
 (segment (start 101.5 100.99) (end 106.63 100.99) (width 0.2) (layer "F.Cu") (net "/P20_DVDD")))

